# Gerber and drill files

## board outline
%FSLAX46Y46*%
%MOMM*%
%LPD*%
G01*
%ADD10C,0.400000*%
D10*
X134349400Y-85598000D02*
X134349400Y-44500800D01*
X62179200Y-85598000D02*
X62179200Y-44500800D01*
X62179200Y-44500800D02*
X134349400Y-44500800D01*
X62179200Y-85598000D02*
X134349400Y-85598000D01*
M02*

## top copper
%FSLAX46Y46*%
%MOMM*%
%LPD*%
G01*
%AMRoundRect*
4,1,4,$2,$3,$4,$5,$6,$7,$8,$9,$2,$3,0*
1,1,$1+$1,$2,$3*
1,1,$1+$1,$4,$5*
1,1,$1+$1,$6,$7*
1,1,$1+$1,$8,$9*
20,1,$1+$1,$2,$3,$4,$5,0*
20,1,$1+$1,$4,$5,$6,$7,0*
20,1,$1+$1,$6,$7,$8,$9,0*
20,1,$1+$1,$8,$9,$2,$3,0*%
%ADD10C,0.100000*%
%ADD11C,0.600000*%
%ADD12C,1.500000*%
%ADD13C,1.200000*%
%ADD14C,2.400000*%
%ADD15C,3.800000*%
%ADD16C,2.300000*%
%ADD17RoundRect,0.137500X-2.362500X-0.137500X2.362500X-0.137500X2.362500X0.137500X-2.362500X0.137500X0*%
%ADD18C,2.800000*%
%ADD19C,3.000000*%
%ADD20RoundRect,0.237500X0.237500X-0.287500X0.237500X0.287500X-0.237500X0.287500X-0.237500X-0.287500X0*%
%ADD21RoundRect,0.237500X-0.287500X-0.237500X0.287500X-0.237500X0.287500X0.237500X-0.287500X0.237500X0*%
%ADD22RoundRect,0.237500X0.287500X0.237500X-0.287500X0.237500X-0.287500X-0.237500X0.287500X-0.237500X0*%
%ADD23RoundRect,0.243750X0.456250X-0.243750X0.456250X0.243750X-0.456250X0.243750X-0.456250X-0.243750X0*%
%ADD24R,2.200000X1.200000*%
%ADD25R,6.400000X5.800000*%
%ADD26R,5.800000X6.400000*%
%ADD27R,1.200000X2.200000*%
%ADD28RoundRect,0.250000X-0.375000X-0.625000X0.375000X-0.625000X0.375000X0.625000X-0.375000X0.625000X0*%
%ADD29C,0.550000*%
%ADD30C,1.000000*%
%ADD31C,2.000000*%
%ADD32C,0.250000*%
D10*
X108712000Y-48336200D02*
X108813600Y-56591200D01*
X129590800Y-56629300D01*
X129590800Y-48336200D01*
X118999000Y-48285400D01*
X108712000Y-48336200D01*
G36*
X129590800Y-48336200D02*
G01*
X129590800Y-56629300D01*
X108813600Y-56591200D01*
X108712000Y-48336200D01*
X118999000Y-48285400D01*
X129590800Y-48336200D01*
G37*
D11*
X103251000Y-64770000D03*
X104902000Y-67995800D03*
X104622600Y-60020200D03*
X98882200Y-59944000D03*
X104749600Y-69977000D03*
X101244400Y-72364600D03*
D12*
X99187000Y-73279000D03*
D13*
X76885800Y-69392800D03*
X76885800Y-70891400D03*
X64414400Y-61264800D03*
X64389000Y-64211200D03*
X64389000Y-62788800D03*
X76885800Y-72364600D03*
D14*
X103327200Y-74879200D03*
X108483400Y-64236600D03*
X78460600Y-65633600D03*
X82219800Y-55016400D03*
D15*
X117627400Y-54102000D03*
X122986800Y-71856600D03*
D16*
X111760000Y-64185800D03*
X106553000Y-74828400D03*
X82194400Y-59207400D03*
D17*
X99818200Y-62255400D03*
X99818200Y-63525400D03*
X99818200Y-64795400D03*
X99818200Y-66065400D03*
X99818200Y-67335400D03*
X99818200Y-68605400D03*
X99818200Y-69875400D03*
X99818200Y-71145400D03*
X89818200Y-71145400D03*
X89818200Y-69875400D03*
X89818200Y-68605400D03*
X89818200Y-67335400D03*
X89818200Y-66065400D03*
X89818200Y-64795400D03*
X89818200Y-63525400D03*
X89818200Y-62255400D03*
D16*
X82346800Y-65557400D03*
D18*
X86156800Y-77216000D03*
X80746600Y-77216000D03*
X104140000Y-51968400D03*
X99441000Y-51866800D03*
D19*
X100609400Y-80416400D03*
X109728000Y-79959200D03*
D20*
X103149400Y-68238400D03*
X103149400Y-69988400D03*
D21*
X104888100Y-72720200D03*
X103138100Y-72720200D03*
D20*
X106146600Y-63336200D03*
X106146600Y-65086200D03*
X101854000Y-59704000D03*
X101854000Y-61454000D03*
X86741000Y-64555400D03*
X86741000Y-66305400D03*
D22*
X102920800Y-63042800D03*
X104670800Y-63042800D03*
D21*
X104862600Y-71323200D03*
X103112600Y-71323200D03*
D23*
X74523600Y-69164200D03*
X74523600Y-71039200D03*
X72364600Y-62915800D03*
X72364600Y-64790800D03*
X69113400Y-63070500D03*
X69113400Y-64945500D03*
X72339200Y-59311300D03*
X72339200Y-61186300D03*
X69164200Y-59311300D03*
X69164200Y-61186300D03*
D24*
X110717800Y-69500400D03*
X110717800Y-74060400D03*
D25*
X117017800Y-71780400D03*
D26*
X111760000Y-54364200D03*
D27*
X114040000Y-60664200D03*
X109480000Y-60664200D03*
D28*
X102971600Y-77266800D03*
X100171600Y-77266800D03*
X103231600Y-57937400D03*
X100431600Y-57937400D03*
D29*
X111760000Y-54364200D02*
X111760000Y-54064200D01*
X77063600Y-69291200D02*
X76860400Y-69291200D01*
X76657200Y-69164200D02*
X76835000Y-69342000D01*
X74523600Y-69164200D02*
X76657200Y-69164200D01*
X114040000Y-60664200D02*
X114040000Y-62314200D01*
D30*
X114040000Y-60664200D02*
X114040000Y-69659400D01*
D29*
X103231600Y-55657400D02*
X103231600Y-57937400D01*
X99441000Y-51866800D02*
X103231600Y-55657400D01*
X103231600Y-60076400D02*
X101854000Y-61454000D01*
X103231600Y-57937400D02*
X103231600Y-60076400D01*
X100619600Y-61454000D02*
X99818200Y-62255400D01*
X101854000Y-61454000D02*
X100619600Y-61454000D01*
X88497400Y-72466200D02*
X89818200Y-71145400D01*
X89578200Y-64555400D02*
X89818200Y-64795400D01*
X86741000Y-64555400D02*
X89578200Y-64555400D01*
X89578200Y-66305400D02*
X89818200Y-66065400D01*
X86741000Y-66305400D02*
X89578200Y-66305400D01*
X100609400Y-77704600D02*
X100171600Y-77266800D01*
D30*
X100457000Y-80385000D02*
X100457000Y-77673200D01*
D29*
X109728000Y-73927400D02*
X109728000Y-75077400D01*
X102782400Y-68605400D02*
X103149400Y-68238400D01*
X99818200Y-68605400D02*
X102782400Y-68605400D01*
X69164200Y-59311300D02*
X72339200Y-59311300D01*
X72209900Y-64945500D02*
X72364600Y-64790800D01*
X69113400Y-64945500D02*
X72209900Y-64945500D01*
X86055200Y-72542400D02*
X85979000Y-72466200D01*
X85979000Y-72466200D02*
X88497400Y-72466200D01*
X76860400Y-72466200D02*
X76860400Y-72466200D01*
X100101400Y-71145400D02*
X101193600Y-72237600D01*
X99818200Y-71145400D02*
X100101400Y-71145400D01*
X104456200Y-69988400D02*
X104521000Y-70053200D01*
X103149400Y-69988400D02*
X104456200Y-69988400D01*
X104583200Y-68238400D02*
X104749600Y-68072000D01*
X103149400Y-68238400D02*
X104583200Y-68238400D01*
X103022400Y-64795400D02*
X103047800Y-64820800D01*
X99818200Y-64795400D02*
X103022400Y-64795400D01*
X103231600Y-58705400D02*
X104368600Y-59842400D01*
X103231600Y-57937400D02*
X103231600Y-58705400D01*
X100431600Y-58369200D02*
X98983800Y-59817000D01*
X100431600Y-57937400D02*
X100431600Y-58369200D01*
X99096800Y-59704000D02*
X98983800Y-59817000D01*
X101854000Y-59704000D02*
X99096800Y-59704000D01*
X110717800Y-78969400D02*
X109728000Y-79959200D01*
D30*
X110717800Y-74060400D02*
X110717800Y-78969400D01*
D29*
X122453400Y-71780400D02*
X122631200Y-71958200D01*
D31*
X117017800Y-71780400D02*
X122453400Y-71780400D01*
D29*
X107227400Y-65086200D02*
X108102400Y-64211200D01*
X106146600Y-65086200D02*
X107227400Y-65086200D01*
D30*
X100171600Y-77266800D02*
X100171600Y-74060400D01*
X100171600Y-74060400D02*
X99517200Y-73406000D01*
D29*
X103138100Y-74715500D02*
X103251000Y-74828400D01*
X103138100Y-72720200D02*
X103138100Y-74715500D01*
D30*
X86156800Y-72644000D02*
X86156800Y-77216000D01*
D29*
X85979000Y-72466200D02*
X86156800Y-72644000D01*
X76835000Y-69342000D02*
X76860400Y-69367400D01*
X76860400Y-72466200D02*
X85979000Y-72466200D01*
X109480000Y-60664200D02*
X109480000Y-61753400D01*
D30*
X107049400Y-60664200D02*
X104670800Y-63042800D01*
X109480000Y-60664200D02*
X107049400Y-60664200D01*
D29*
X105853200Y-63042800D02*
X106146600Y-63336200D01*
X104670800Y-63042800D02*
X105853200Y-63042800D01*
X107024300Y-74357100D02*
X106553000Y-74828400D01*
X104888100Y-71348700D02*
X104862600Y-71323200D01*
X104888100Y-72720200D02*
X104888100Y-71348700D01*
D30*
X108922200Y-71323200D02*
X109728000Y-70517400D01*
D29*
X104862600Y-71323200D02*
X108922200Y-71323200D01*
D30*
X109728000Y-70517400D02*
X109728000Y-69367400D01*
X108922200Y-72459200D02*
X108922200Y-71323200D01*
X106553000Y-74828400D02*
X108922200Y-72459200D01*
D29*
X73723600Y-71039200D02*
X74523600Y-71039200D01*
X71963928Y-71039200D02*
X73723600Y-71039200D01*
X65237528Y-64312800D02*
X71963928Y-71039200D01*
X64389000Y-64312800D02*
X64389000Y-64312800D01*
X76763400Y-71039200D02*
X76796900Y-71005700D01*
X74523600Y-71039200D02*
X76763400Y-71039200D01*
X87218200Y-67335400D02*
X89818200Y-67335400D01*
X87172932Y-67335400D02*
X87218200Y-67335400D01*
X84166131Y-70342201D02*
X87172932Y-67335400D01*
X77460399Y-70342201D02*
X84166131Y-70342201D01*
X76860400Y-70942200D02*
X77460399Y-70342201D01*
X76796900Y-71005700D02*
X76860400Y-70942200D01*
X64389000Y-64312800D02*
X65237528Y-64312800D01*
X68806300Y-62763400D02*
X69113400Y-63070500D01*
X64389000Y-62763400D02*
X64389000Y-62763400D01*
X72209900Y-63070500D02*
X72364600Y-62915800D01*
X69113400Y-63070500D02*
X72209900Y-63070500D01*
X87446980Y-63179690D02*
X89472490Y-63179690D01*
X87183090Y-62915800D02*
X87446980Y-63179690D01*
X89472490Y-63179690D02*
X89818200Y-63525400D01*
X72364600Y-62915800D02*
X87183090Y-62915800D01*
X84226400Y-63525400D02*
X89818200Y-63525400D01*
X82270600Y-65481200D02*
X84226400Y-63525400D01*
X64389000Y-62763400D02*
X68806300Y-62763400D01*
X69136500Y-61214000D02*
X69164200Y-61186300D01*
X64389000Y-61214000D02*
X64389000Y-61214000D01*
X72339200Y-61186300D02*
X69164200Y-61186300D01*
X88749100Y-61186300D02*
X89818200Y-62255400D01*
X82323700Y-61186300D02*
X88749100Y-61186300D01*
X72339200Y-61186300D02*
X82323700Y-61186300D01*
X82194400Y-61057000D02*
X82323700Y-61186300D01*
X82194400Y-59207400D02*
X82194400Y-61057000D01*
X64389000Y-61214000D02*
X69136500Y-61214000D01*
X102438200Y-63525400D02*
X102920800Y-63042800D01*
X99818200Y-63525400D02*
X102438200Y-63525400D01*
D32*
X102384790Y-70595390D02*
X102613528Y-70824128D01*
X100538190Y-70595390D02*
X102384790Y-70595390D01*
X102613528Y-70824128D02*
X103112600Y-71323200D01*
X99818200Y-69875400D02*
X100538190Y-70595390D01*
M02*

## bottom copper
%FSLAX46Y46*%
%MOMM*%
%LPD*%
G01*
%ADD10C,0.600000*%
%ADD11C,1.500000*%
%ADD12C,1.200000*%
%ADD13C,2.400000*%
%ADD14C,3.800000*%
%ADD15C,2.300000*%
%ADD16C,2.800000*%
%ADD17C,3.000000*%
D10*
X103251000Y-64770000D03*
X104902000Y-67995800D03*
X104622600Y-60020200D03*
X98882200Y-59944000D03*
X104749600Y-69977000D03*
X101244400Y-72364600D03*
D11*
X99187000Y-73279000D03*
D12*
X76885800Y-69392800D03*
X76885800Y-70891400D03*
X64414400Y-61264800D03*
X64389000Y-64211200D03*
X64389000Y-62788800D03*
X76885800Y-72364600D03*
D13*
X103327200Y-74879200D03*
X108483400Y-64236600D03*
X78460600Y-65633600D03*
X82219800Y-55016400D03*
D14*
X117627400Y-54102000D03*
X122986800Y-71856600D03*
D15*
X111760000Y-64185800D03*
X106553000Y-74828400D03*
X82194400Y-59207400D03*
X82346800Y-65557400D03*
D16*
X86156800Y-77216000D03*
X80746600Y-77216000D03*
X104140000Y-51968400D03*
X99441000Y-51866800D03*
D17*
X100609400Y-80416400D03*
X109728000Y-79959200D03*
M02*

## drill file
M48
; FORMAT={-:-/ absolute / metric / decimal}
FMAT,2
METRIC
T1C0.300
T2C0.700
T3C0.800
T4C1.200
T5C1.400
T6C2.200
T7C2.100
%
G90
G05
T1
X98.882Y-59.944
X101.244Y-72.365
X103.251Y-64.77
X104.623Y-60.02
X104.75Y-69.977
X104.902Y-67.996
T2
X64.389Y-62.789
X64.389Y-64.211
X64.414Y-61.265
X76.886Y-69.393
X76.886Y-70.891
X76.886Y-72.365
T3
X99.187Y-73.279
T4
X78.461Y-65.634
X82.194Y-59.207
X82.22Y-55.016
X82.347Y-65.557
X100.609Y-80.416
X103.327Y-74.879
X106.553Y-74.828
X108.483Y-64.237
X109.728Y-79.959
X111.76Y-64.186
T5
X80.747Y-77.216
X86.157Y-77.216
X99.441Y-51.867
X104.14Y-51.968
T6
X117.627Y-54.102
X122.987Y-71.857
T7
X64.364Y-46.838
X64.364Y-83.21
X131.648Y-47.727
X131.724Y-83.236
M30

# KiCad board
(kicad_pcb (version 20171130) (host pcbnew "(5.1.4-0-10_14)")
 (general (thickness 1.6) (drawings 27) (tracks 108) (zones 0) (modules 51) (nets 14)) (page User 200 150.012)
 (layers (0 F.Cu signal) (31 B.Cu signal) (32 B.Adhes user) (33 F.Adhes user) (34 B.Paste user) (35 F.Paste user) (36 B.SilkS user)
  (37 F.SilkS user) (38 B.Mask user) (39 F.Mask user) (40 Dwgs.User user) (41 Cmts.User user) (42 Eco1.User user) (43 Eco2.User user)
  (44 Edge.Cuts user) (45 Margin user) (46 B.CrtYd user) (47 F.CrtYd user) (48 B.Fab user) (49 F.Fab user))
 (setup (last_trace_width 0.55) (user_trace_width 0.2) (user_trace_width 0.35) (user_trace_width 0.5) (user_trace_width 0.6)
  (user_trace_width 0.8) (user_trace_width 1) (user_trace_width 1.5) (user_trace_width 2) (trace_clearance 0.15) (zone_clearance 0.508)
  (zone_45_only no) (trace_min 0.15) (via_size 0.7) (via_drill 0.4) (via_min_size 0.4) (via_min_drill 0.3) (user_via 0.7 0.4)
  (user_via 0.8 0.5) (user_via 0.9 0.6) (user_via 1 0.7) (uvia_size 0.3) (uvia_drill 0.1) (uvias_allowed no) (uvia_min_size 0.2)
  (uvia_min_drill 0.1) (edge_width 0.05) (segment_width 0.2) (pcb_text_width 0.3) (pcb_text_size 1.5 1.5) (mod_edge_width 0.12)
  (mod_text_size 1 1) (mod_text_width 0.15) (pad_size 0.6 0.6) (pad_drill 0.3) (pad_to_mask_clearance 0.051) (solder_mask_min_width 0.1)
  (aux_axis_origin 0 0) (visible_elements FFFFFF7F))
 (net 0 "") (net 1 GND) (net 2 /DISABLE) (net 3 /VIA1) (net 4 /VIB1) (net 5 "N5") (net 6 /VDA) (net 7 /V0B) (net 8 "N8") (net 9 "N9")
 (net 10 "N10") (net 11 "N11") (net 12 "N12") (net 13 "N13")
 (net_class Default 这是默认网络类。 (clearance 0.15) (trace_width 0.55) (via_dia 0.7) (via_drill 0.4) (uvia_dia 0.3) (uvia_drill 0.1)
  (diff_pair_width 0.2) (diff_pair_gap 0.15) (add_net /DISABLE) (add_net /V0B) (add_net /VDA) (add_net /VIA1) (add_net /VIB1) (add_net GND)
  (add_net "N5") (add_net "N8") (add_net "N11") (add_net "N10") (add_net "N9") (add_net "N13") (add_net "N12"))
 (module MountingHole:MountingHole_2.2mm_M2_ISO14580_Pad (layer F.Cu) (at 103.251 64.77)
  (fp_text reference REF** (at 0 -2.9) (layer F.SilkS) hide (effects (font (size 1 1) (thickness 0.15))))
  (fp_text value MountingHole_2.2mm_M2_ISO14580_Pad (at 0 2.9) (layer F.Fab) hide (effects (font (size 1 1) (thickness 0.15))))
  (pad 1 thru_hole circle (at 0 0) (size 0.6 0.6) (drill 0.3) (layers *.Cu *.Mask) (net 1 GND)))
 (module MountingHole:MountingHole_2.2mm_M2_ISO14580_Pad (layer F.Cu) (at 104.902 67.9958)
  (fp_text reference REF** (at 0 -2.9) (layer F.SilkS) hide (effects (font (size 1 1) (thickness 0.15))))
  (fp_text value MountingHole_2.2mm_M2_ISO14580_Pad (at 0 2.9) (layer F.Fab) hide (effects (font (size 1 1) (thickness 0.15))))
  (pad 1 thru_hole circle (at 0 0) (size 0.6 0.6) (drill 0.3) (layers *.Cu *.Mask) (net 1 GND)))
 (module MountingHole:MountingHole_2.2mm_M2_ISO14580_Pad (layer F.Cu) (at 104.6226 60.0202)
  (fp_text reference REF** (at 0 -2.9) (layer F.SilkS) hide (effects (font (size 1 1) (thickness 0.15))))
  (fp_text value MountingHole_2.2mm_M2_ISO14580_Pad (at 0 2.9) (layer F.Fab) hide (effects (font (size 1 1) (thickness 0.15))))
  (pad 1 thru_hole circle (at 0 0) (size 0.6 0.6) (drill 0.3) (layers *.Cu *.Mask) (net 1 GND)))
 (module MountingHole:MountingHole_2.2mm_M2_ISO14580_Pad (layer F.Cu) (at 98.8822 59.944)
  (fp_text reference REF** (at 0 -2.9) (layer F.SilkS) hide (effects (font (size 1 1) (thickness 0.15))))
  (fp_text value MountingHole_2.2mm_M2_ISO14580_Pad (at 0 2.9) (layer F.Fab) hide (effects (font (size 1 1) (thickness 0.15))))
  (pad 1 thru_hole circle (at 0 0) (size 0.6 0.6) (drill 0.3) (layers *.Cu *.Mask) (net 1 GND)))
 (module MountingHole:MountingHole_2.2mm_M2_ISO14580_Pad (layer F.Cu) (at 104.7496 69.977)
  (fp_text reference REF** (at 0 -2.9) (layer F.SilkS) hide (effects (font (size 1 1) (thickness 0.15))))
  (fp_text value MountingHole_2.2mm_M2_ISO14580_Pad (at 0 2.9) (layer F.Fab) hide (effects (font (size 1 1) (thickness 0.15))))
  (pad 1 thru_hole circle (at 0 0) (size 0.6 0.6) (drill 0.3) (layers *.Cu *.Mask) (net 1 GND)))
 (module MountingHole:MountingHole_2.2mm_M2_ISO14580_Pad (layer F.Cu) (at 101.2444 72.3646)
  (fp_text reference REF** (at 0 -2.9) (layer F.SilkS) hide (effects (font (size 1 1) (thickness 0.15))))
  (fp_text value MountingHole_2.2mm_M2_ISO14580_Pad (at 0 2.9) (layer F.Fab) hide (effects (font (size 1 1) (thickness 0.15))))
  (pad 1 thru_hole circle (at 0 0) (size 0.6 0.6) (drill 0.3) (layers *.Cu *.Mask) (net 1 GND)))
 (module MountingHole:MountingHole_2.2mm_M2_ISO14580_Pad (layer F.Cu) (at 99.187 73.279)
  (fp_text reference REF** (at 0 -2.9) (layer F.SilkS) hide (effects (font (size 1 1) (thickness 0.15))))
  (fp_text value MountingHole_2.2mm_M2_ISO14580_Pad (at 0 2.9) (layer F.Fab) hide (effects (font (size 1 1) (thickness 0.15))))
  (pad 1 thru_hole circle (at 0 0) (size 1.5 1.5) (drill 0.8) (layers *.Cu *.Mask) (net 1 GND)))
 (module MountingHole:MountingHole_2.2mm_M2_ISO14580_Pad (layer F.Cu) (at 76.8858 69.3928)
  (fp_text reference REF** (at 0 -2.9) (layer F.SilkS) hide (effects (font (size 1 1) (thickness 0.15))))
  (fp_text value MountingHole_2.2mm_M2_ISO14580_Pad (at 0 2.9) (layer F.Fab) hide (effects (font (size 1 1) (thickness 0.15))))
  (pad 1 thru_hole circle (at 0 0) (size 1.2 1.2) (drill 0.7) (layers *.Cu *.Mask) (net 1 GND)))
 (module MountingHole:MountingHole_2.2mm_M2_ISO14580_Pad (layer F.Cu) (at 76.8858 70.8914)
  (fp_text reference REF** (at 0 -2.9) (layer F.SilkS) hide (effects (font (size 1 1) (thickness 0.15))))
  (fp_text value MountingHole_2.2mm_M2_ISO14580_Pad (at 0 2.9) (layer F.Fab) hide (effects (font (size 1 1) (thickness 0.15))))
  (pad 1 thru_hole circle (at 0 0) (size 1.2 1.2) (drill 0.7) (layers *.Cu *.Mask) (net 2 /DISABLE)))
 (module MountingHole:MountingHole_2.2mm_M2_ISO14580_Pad (layer F.Cu) (at 64.4144 61.2648)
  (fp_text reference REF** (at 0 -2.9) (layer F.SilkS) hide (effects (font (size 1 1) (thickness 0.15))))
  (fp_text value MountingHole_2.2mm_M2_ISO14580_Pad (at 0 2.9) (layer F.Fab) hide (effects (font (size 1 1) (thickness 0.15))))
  (pad 1 thru_hole circle (at 0 0) (size 1.2 1.2) (drill 0.7) (layers *.Cu *.Mask) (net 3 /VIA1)))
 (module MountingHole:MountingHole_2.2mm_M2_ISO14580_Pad (layer F.Cu) (at 64.389 64.2112)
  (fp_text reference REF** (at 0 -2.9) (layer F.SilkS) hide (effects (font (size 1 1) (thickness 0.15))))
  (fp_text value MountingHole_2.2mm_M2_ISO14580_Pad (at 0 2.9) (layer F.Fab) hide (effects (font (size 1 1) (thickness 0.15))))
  (pad 1 thru_hole circle (at 0 0) (size 1.2 1.2) (drill 0.7) (layers *.Cu *.Mask) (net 2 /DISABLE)))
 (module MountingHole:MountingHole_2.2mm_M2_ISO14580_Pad (layer F.Cu) (at 64.389 62.7888)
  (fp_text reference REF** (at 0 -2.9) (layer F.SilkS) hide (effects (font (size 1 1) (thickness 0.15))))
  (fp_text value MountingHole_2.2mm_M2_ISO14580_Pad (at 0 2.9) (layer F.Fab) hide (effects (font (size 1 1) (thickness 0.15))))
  (pad 1 thru_hole circle (at 0 0) (size 1.2 1.2) (drill 0.7) (layers *.Cu *.Mask) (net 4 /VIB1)))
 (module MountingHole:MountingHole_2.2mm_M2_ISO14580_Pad (layer F.Cu) (at 76.8858 72.3646)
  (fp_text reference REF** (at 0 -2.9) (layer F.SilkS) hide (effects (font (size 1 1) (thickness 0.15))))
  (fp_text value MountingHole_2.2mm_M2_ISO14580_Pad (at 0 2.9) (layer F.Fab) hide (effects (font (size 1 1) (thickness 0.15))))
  (pad 1 thru_hole circle (at 0 0) (size 1.2 1.2) (drill 0.7) (layers *.Cu *.Mask) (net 1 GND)))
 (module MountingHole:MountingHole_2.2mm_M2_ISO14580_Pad (layer F.Cu) (at 103.3272 74.8792)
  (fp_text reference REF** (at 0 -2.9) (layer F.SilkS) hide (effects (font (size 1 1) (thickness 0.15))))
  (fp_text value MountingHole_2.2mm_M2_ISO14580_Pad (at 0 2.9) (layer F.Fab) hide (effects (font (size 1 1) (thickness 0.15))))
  (pad 1 thru_hole circle (at 0 0) (size 2.4 2.4) (drill 1.2) (layers *.Cu *.Mask) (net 1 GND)))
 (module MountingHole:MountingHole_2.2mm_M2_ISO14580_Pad (layer F.Cu) (at 108.4834 64.2366)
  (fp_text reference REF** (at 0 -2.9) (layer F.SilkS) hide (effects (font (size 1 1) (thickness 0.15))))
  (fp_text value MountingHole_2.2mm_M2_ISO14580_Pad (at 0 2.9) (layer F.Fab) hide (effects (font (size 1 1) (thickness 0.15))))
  (pad 1 thru_hole circle (at 0 0) (size 2.4 2.4) (drill 1.2) (layers *.Cu *.Mask) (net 1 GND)))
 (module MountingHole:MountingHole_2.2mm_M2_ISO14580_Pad (layer F.Cu) (at 78.4606 65.6336)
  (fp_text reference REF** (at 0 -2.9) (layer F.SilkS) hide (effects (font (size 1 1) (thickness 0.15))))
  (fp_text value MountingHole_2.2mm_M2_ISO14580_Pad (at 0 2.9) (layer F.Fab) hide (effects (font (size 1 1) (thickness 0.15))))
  (pad 1 thru_hole circle (at 0 0) (size 2.4 2.4) (drill 1.2) (layers *.Cu *.Mask) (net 1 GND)))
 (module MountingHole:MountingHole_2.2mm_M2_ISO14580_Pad (layer F.Cu) (at 82.2198 55.0164)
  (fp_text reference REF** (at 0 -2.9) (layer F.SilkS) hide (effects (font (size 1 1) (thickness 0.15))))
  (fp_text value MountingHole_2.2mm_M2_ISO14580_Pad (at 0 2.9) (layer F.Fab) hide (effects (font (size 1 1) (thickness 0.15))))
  (pad 1 thru_hole circle (at 0 0) (size 2.4 2.4) (drill 1.2) (layers *.Cu *.Mask) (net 1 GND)))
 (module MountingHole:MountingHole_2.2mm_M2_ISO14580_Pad (layer F.Cu) (at 117.6274 54.102)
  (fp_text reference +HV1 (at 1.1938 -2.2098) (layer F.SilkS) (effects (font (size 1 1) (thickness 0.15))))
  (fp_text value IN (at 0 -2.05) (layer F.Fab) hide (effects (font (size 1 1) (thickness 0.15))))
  (pad 1 thru_hole circle (at 0 0) (size 3.8 3.8) (drill 2.2) (layers *.Cu *.Mask) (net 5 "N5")))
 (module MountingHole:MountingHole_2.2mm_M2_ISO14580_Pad (layer F.Cu) (at 122.9868 71.8566)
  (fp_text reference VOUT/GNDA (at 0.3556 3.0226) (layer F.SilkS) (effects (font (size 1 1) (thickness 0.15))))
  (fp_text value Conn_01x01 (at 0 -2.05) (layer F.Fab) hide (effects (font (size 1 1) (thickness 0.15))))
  (pad 1 thru_hole circle (at 0 0) (size 3.8 3.8) (drill 2.2) (layers *.Cu *.Mask) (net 1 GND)))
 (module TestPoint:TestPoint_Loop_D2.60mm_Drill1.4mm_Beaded (layer F.Cu) (at 111.76 64.1858)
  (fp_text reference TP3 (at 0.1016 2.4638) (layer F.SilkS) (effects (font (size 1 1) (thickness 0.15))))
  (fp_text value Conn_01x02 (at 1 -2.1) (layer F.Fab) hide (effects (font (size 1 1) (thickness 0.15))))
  (pad 1 thru_hole circle (at 0 0) (size 2.3 2.3) (drill 1.2) (layers *.Cu *.Mask) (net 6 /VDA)))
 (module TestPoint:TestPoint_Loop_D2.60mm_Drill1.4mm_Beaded (layer F.Cu) (at 106.553 74.8284)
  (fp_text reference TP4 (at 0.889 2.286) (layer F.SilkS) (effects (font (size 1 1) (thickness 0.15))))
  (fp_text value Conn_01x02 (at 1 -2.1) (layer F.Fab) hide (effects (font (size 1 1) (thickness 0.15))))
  (pad 1 thru_hole circle (at 0 0) (size 2.3 2.3) (drill 1.2) (layers *.Cu *.Mask) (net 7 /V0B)))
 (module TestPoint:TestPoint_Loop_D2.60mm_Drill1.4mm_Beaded (layer F.Cu) (at 82.1944 59.2074 90)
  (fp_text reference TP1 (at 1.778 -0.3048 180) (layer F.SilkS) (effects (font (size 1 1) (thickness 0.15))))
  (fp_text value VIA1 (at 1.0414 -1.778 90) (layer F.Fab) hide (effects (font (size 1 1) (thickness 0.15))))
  (pad 1 thru_hole circle (at 0 0 90) (size 2.3 2.3) (drill 1.2) (layers *.Cu *.Mask) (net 3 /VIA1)))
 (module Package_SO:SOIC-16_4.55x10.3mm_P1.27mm (layer F.Cu) (at 94.8182 66.7004)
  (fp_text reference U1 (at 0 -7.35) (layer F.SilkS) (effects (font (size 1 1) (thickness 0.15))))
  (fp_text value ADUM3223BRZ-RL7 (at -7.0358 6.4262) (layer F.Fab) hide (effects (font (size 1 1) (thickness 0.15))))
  (pad 16 smd roundrect (at 5 -4.445) (size 5 0.55) (layers F.Cu F.Paste F.Mask) (roundrect_rratio 0.25) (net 1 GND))
  (pad 15 smd roundrect (at 5 -3.175) (size 5 0.55) (layers F.Cu F.Paste F.Mask) (roundrect_rratio 0.25) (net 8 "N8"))
  (pad 14 smd roundrect (at 5 -1.905) (size 5 0.55) (layers F.Cu F.Paste F.Mask) (roundrect_rratio 0.25) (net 1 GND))
  (pad 13 smd roundrect (at 5 -0.635) (size 5 0.55) (layers F.Cu F.Paste F.Mask) (roundrect_rratio 0.25) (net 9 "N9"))
  (pad 12 smd roundrect (at 5 0.635) (size 5 0.55) (layers F.Cu F.Paste F.Mask) (roundrect_rratio 0.25) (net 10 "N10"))
  (pad 11 smd roundrect (at 5 1.905) (size 5 0.55) (layers F.Cu F.Paste F.Mask) (roundrect_rratio 0.25) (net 1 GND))
  (pad 10 smd roundrect (at 5 3.175) (size 5 0.55) (layers F.Cu F.Paste F.Mask) (roundrect_rratio 0.25) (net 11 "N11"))
  (pad 9 smd roundrect (at 5 4.445) (size 5 0.55) (layers F.Cu F.Paste F.Mask) (roundrect_rratio 0.25) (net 1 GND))
  (pad 8 smd roundrect (at -5 4.445) (size 5 0.55) (layers F.Cu F.Paste F.Mask) (roundrect_rratio 0.25) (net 1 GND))
  (pad 7 smd roundrect (at -5 3.175) (size 5 0.55) (layers F.Cu F.Paste F.Mask) (roundrect_rratio 0.25) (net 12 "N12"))
  (pad 6 smd roundrect (at -5 1.905) (size 5 0.55) (layers F.Cu F.Paste F.Mask) (roundrect_rratio 0.25) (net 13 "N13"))
  (pad 5 smd roundrect (at -5 0.635) (size 5 0.55) (layers F.Cu F.Paste F.Mask) (roundrect_rratio 0.25) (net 2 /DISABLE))
  (pad 4 smd roundrect (at -5 -0.635) (size 5 0.55) (layers F.Cu F.Paste F.Mask) (roundrect_rratio 0.25) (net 1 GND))
  (pad 3 smd roundrect (at -5 -1.905) (size 5 0.55) (layers F.Cu F.Paste F.Mask) (roundrect_rratio 0.25) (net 1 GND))
  (pad 2 smd roundrect (at -5 -3.175) (size 5 0.55) (layers F.Cu F.Paste F.Mask) (roundrect_rratio 0.25) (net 4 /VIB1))
  (pad 1 smd roundrect (at -5 -4.445) (size 5 0.55) (layers F.Cu F.Paste F.Mask) (roundrect_rratio 0.25) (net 3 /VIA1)))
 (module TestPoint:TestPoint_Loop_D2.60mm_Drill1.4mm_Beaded (layer F.Cu) (at 82.3468 65.5574 180)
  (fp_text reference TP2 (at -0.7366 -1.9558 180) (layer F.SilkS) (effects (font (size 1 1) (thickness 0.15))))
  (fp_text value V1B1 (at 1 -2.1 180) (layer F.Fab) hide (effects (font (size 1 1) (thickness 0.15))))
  (pad 1 thru_hole circle (at 0 0 180) (size 2.3 2.3) (drill 1.2) (layers *.Cu *.Mask) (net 4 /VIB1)))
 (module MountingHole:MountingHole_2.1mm (layer F.Cu) (at 131.6482 47.7266)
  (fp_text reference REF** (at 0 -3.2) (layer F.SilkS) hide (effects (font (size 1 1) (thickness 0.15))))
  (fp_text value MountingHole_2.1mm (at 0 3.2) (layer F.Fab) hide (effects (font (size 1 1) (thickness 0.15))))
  (pad "" np_thru_hole circle (at 0 0) (size 2.1 2.1) (drill 2.1) (layers *.Cu *.Mask)))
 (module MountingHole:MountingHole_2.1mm (layer F.Cu) (at 131.7752 83.2358)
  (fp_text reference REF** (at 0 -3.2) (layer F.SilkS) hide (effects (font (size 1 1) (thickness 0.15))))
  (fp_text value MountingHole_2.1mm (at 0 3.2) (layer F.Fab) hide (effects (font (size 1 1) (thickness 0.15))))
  (pad "" np_thru_hole circle (at -0.0508 0) (size 2.1 2.1) (drill 2.1) (layers *.Cu *.Mask)))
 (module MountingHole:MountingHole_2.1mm (layer F.Cu) (at 64.3636 83.2104)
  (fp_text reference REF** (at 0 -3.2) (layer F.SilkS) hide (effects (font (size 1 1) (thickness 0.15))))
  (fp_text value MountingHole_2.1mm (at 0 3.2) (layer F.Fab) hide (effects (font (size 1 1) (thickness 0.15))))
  (pad "" np_thru_hole circle (at 0 0) (size 2.1 2.1) (drill 2.1) (layers *.Cu *.Mask)))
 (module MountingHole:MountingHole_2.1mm (layer F.Cu) (at 64.3636 46.8376)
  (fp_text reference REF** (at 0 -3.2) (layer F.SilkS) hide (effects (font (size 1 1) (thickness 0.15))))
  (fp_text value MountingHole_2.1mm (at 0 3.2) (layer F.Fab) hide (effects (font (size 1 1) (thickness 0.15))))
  (pad "" np_thru_hole circle (at 0 0) (size 2.1 2.1) (drill 2.1) (layers *.Cu *.Mask)))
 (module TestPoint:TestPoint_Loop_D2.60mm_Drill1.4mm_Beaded (layer F.Cu) (at 86.1568 77.216)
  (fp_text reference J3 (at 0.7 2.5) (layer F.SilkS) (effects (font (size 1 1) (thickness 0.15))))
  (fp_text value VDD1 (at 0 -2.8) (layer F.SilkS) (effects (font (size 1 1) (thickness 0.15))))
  (pad 1 thru_hole circle (at 0 0) (size 2.8 2.8) (drill 1.4) (layers *.Cu *.Mask) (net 1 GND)))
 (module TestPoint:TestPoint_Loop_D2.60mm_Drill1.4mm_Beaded (layer F.Cu) (at 80.7466 77.216)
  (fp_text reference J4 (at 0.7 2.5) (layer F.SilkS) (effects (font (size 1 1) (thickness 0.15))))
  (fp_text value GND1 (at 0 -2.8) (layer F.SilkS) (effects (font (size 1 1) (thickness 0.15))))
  (pad 1 thru_hole circle (at 0 0) (size 2.8 2.8) (drill 1.4) (layers *.Cu *.Mask) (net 1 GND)))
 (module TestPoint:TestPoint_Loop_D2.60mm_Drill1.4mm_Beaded (layer F.Cu) (at 104.14 51.9684)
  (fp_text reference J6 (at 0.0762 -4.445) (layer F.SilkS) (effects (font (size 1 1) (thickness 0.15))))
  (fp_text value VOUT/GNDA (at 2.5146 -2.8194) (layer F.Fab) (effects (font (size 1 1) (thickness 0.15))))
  (pad 1 thru_hole circle (at 0 0) (size 2.8 2.8) (drill 1.4) (layers *.Cu *.Mask)))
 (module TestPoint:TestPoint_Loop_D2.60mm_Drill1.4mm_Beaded (layer F.Cu) (at 99.441 51.8668)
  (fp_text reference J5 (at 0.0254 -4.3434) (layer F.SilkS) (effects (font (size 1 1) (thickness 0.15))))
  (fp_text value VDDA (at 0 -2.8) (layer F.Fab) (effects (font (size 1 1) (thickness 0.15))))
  (pad 1 thru_hole circle (at 0 0) (size 2.8 2.8) (drill 1.4) (layers *.Cu *.Mask) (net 1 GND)))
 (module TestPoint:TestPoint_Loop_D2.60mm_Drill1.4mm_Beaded (layer F.Cu) (at 100.6094 80.4164)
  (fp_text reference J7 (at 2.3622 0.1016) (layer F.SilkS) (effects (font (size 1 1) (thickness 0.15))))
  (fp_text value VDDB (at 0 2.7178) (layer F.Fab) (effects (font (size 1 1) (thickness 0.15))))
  (pad 1 thru_hole circle (at 0 0) (size 3 3) (drill 1.2) (layers *.Cu *.Mask) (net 1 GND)))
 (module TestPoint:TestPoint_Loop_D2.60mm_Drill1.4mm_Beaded (layer F.Cu) (at 109.728 79.9592)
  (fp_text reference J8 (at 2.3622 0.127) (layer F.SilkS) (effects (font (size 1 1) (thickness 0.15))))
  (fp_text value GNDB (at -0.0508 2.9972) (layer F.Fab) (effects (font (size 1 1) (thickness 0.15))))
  (pad 1 thru_hole circle (at 0 0) (size 3 3) (drill 1.2) (layers *.Cu *.Mask) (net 1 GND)))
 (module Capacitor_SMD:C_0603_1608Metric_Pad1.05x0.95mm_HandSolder (layer F.Cu) (at 103.1494 69.1134 90)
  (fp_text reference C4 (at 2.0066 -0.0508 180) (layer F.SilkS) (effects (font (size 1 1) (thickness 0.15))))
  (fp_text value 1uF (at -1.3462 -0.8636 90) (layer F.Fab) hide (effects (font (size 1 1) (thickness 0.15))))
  (pad 2 smd roundrect (at 0.875 0 90) (size 1.05 0.95) (layers F.Cu F.Paste F.Mask) (roundrect_rratio 0.25) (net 1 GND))
  (pad 1 smd roundrect (at -0.875 0 90) (size 1.05 0.95) (layers F.Cu F.Paste F.Mask) (roundrect_rratio 0.25) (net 1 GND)))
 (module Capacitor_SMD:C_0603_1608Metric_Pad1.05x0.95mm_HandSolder (layer F.Cu) (at 104.0131 72.7202)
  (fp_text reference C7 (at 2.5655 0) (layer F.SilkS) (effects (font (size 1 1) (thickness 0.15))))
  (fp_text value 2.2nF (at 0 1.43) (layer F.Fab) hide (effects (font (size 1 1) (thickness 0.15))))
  (pad 2 smd roundrect (at 0.875 0) (size 1.05 0.95) (layers F.Cu F.Paste F.Mask) (roundrect_rratio 0.25) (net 7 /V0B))
  (pad 1 smd roundrect (at -0.875 0) (size 1.05 0.95) (layers F.Cu F.Paste F.Mask) (roundrect_rratio 0.25) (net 1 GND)))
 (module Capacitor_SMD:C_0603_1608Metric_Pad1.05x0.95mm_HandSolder (layer F.Cu) (at 106.1466 64.2112 90)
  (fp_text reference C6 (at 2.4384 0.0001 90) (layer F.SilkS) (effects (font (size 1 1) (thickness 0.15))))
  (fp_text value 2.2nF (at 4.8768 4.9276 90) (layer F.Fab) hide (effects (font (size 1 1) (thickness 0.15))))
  (pad 2 smd roundrect (at 0.875 0 90) (size 1.05 0.95) (layers F.Cu F.Paste F.Mask) (roundrect_rratio 0.25) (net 6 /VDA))
  (pad 1 smd roundrect (at -0.875 0 90) (size 1.05 0.95) (layers F.Cu F.Paste F.Mask) (roundrect_rratio 0.25) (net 1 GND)))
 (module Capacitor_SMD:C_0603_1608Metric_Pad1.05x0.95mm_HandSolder (layer F.Cu) (at 101.854 60.579 90)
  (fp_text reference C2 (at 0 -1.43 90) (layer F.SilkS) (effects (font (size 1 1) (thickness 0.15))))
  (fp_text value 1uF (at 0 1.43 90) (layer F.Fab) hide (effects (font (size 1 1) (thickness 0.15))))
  (pad 2 smd roundrect (at 0.875 0 90) (size 1.05 0.95) (layers F.Cu F.Paste F.Mask) (roundrect_rratio 0.25) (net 1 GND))
  (pad 1 smd roundrect (at -0.875 0 90) (size 1.05 0.95) (layers F.Cu F.Paste F.Mask) (roundrect_rratio 0.25) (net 1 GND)))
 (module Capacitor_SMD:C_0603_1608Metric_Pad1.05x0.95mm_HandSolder (layer F.Cu) (at 86.741 65.4304 90)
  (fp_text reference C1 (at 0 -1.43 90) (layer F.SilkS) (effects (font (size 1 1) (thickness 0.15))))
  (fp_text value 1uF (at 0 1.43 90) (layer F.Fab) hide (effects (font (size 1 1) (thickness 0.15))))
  (pad 2 smd roundrect (at 0.875 0 90) (size 1.05 0.95) (layers F.Cu F.Paste F.Mask) (roundrect_rratio 0.25) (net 1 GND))
  (pad 1 smd roundrect (at -0.875 0 90) (size 1.05 0.95) (layers F.Cu F.Paste F.Mask) (roundrect_rratio 0.25) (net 1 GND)))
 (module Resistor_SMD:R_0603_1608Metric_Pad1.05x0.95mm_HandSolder (layer F.Cu) (at 103.7958 63.0428 180)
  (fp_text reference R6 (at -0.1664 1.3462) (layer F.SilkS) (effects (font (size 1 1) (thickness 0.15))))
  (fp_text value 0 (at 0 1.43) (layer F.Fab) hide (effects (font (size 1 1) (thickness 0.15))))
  (pad 2 smd roundrect (at 0.875 0 180) (size 1.05 0.95) (layers F.Cu F.Paste F.Mask) (roundrect_rratio 0.25) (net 8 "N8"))
  (pad 1 smd roundrect (at -0.875 0 180) (size 1.05 0.95) (layers F.Cu F.Paste F.Mask) (roundrect_rratio 0.25) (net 6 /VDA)))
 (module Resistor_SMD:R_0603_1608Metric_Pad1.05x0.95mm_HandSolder (layer F.Cu) (at 103.9876 71.3232)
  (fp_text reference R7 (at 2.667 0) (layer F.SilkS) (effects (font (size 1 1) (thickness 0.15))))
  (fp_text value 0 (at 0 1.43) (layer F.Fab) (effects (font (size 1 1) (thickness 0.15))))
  (pad 2 smd roundrect (at 0.875 0) (size 1.05 0.95) (layers F.Cu F.Paste F.Mask) (roundrect_rratio 0.25) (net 7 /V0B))
  (pad 1 smd roundrect (at -0.875 0) (size 1.05 0.95) (layers F.Cu F.Paste F.Mask) (roundrect_rratio 0.25) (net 11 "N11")))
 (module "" (layer F.Cu) (at 64.7446 49.2506 90)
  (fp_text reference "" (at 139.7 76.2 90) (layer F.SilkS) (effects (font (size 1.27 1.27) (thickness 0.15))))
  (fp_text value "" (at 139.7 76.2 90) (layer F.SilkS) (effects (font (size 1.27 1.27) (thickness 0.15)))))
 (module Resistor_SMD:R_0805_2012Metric (layer F.Cu) (at 74.5236 70.1017 90)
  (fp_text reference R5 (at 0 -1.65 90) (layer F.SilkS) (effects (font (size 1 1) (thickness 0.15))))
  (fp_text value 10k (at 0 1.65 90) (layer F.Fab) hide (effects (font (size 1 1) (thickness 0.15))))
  (pad 2 smd roundrect (at 0.9375 0 90) (size 0.975 1.4) (layers F.Cu F.Paste F.Mask) (roundrect_rratio 0.25) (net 1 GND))
  (pad 1 smd roundrect (at -0.9375 0 90) (size 0.975 1.4) (layers F.Cu F.Paste F.Mask) (roundrect_rratio 0.25) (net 2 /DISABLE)))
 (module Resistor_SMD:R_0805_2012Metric (layer F.Cu) (at 72.3646 63.8533 90)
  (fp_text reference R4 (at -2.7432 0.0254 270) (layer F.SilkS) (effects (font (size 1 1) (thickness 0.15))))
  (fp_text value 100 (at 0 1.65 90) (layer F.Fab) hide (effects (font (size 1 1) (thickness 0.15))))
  (pad 2 smd roundrect (at 0.9375 0 90) (size 0.975 1.4) (layers F.Cu F.Paste F.Mask) (roundrect_rratio 0.25) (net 4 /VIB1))
  (pad 1 smd roundrect (at -0.9375 0 90) (size 0.975 1.4) (layers F.Cu F.Paste F.Mask) (roundrect_rratio 0.25) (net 1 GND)))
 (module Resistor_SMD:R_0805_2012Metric (layer F.Cu) (at 69.1134 64.008 90)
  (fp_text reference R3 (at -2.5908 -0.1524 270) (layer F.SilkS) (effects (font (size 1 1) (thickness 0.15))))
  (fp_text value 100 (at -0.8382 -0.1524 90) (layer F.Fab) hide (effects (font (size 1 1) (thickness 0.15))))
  (pad 2 smd roundrect (at 0.9375 0 90) (size 0.975 1.4) (layers F.Cu F.Paste F.Mask) (roundrect_rratio 0.25) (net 4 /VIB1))
  (pad 1 smd roundrect (at -0.9375 0 90) (size 0.975 1.4) (layers F.Cu F.Paste F.Mask) (roundrect_rratio 0.25) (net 1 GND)))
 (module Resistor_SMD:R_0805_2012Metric (layer F.Cu) (at 72.3392 60.2488 90)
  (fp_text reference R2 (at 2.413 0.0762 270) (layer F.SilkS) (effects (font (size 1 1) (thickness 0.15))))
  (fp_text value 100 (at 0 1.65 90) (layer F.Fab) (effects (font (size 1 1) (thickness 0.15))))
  (pad 2 smd roundrect (at 0.9375 0 90) (size 0.975 1.4) (layers F.Cu F.Paste F.Mask) (roundrect_rratio 0.25) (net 1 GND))
  (pad 1 smd roundrect (at -0.9375 0 90) (size 0.975 1.4) (layers F.Cu F.Paste F.Mask) (roundrect_rratio 0.25) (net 3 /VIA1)))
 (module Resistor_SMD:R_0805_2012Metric (layer F.Cu) (at 69.1642 60.2488 90)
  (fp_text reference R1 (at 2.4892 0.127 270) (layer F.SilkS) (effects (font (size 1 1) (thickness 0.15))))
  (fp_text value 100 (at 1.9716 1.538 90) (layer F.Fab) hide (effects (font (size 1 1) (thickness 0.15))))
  (pad 2 smd roundrect (at 0.9375 0 90) (size 0.975 1.4) (layers F.Cu F.Paste F.Mask) (roundrect_rratio 0.25) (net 1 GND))
  (pad 1 smd roundrect (at -0.9375 0 90) (size 0.975 1.4) (layers F.Cu F.Paste F.Mask) (roundrect_rratio 0.25) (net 3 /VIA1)))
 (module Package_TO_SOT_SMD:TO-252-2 (layer F.Cu) (at 114.9178 71.7804)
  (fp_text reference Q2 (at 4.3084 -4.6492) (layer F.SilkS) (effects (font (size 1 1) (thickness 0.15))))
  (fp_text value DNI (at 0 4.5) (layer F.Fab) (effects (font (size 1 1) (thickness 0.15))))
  (pad 1 smd rect (at -4.2 -2.28) (size 2.2 1.2) (layers F.Cu F.Paste F.Mask) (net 7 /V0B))
  (pad 3 smd rect (at -4.2 2.28) (size 2.2 1.2) (layers F.Cu F.Paste F.Mask) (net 1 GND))
  (pad "" smd rect (at 2.1 0) (size 6.4 5.8) (layers F.Cu F.Paste F.Mask))
  (pad "" smd rect (at 3.775 1.525) (size 3.05 2.75) (layers F.Paste))
  (pad "" smd rect (at 0.425 -1.525) (size 3.05 2.75) (layers F.Paste))
  (pad "" smd rect (at 3.775 -1.525) (size 3.05 2.75) (layers F.Paste))
  (pad "" smd rect (at 0.425 1.525) (size 3.05 2.75) (layers F.Paste)))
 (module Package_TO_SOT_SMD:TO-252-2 (layer F.Cu) (at 111.76 56.4642 90)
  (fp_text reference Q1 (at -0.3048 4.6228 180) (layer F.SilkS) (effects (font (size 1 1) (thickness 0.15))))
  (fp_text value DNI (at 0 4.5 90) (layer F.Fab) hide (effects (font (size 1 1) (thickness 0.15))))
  (pad "" smd rect (at 0.425 1.525 90) (size 3.05 2.75) (layers F.Paste))
  (pad "" smd rect (at 3.775 -1.525 90) (size 3.05 2.75) (layers F.Paste))
  (pad "" smd rect (at 0.425 -1.525 90) (size 3.05 2.75) (layers F.Paste))
  (pad "" smd rect (at 3.775 1.525 90) (size 3.05 2.75) (layers F.Paste))
  (pad 2 smd rect (at 2.1 0 90) (size 6.4 5.8) (layers F.Cu F.Mask))
  (pad 3 smd rect (at -4.2 2.28 90) (size 2.2 1.2) (layers F.Cu F.Paste F.Mask) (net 1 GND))
  (pad 1 smd rect (at -4.2 -2.28 90) (size 2.2 1.2) (layers F.Cu F.Paste F.Mask) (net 6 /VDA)))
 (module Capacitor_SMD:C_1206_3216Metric (layer F.Cu) (at 101.5716 77.2668)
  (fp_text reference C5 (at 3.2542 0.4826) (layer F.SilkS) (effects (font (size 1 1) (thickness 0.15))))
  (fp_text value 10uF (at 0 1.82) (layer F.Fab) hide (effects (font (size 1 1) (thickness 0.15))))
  (pad 2 smd roundrect (at 1.4 0) (size 1.25 1.75) (layers F.Cu F.Paste F.Mask) (roundrect_rratio 0.2))
  (pad 1 smd roundrect (at -1.4 0) (size 1.25 1.75) (layers F.Cu F.Paste F.Mask) (roundrect_rratio 0.2) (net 1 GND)))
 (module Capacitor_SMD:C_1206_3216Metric (layer F.Cu) (at 101.8316 57.9374)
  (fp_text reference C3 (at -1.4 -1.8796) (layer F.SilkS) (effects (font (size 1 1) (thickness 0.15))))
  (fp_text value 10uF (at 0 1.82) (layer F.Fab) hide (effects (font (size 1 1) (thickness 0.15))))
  (pad 2 smd roundrect (at 1.4 0) (size 1.25 1.75) (layers F.Cu F.Paste F.Mask) (roundrect_rratio 0.2) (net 1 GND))
  (pad 1 smd roundrect (at -1.4 0) (size 1.25 1.75) (layers F.Cu F.Paste F.Mask) (roundrect_rratio 0.2) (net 1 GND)))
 (gr_line (start 134.3494 85.598) (end 134.3494 44.5008) (layer Edge.Cuts) (width 0.4))
 (gr_line (start 62.1792 85.598) (end 62.1792 44.5008) (layer Edge.Cuts) (width 0.4))
 (gr_line (start 62.1792 44.5008) (end 134.3494 44.5008) (layer Edge.Cuts) (width 0.4))
 (gr_poly
  (pts (xy 108.712 48.3362) (xy 108.8136 56.5912) (xy 129.5908 56.6293) (xy 129.5908 48.3362) (xy 118.999 48.2854)) (layer F.Cu) (width 0.1))
 (gr_line (start 62.1792 85.598) (end 134.3494 85.598) (layer Edge.Cuts) (width 0.4))
 (segment (start 111.76 54.3642) (end 111.76 54.0642) (width 0.55) (layer F.Cu) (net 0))
 (segment (start 77.0636 69.2912) (end 76.8604 69.2912) (width 0.55) (layer F.Cu) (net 1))
 (segment (start 76.6572 69.1642) (end 76.835 69.342) (width 0.55) (layer F.Cu) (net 1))
 (segment (start 74.5236 69.1642) (end 76.6572 69.1642) (width 0.55) (layer F.Cu) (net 1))
 (segment (start 114.04 60.6642) (end 114.04 62.3142) (width 0.55) (layer F.Cu) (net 1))
 (segment (start 114.04 60.6642) (end 114.04 69.6594) (width 1) (layer F.Cu) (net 1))
 (segment (start 103.2316 55.6574) (end 103.2316 57.9374) (width 0.55) (layer F.Cu) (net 1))
 (segment (start 99.441 51.8668) (end 103.2316 55.6574) (width 0.55) (layer F.Cu) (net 1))
 (segment (start 103.2316 60.0764) (end 101.854 61.454) (width 0.55) (layer F.Cu) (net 1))
 (segment (start 103.2316 57.9374) (end 103.2316 60.0764) (width 0.55) (layer F.Cu) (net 1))
 (segment (start 100.6196 61.454) (end 99.8182 62.2554) (width 0.55) (layer F.Cu) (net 1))
 (segment (start 101.854 61.454) (end 100.6196 61.454) (width 0.55) (layer F.Cu) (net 1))
 (segment (start 88.4974 72.4662) (end 89.8182 71.1454) (width 0.55) (layer F.Cu) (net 1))
 (segment (start 89.5782 64.5554) (end 89.8182 64.7954) (width 0.55) (layer F.Cu) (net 1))
 (segment (start 86.741 64.5554) (end 89.5782 64.5554) (width 0.55) (layer F.Cu) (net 1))
 (segment (start 89.5782 66.3054) (end 89.8182 66.0654) (width 0.55) (layer F.Cu) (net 1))
 (segment (start 86.741 66.3054) (end 89.5782 66.3054) (width 0.55) (layer F.Cu) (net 1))
 (segment (start 100.6094 77.7046) (end 100.1716 77.2668) (width 0.55) (layer F.Cu) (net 1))
 (segment (start 100.457 80.385) (end 100.457 77.6732) (width 1) (layer F.Cu) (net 1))
 (segment (start 109.728 73.9274) (end 109.728 75.0774) (width 0.55) (layer F.Cu) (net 1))
 (segment (start 102.7824 68.6054) (end 103.1494 68.2384) (width 0.55) (layer F.Cu) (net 1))
 (segment (start 99.8182 68.6054) (end 102.7824 68.6054) (width 0.55) (layer F.Cu) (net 1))
 (segment (start 69.1642 59.3113) (end 72.3392 59.3113) (width 0.55) (layer F.Cu) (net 1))
 (segment (start 72.2099 64.9455) (end 72.3646 64.7908) (width 0.55) (layer F.Cu) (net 1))
 (segment (start 69.1134 64.9455) (end 72.2099 64.9455) (width 0.55) (layer F.Cu) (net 1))
 (segment (start 86.0552 72.5424) (end 85.979 72.4662) (width 0.55) (layer F.Cu) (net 1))
 (segment (start 85.979 72.4662) (end 88.4974 72.4662) (width 0.55) (layer F.Cu) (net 1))
 (segment (start 76.8604 72.4662) (end 76.8604 72.4662) (width 0.55) (layer F.Cu) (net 1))
 (segment (start 100.1014 71.1454) (end 101.1936 72.2376) (width 0.55) (layer F.Cu) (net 1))
 (segment (start 99.8182 71.1454) (end 100.1014 71.1454) (width 0.55) (layer F.Cu) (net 1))
 (segment (start 104.4562 69.9884) (end 104.521 70.0532) (width 0.55) (layer F.Cu) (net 1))
 (segment (start 103.1494 69.9884) (end 104.4562 69.9884) (width 0.55) (layer F.Cu) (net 1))
 (segment (start 104.5832 68.2384) (end 104.7496 68.072) (width 0.55) (layer F.Cu) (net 1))
 (segment (start 103.1494 68.2384) (end 104.5832 68.2384) (width 0.55) (layer F.Cu) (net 1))
 (segment (start 103.0224 64.7954) (end 103.0478 64.8208) (width 0.55) (layer F.Cu) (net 1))
 (segment (start 99.8182 64.7954) (end 103.0224 64.7954) (width 0.55) (layer F.Cu) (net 1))
 (segment (start 103.2316 58.7054) (end 104.3686 59.8424) (width 0.55) (layer F.Cu) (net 1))
 (segment (start 103.2316 57.9374) (end 103.2316 58.7054) (width 0.55) (layer F.Cu) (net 1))
 (segment (start 100.4316 58.3692) (end 98.9838 59.817) (width 0.55) (layer F.Cu) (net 1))
 (segment (start 100.4316 57.9374) (end 100.4316 58.3692) (width 0.55) (layer F.Cu) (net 1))
 (segment (start 99.0968 59.704) (end 98.9838 59.817) (width 0.55) (layer F.Cu) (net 1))
 (segment (start 101.854 59.704) (end 99.0968 59.704) (width 0.55) (layer F.Cu) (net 1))
 (segment (start 110.7178 78.9694) (end 109.728 79.9592) (width 0.55) (layer F.Cu) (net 1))
 (segment (start 110.7178 74.0604) (end 110.7178 78.9694) (width 1) (layer F.Cu) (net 1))
 (segment (start 122.4534 71.7804) (end 122.6312 71.9582) (width 0.55) (layer F.Cu) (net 1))
 (segment (start 117.0178 71.7804) (end 122.4534 71.7804) (width 2) (layer F.Cu) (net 1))
 (segment (start 107.2274 65.0862) (end 108.1024 64.2112) (width 0.55) (layer F.Cu) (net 1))
 (segment (start 106.1466 65.0862) (end 107.2274 65.0862) (width 0.55) (layer F.Cu) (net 1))
 (segment (start 100.1716 77.2668) (end 100.1716 74.0604) (width 1) (layer F.Cu) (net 1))
 (segment (start 100.1716 74.0604) (end 99.5172 73.406) (width 1) (layer F.Cu) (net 1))
 (segment (start 103.1381 74.7155) (end 103.251 74.8284) (width 0.55) (layer F.Cu) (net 1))
 (segment (start 103.1381 72.7202) (end 103.1381 74.7155) (width 0.55) (layer F.Cu) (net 1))
 (segment (start 86.1568 72.644) (end 86.1568 77.216) (width 1) (layer F.Cu) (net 1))
 (segment (start 85.979 72.4662) (end 86.1568 72.644) (width 0.55) (layer F.Cu) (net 1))
 (segment (start 76.835 69.342) (end 76.8604 69.3674) (width 0.55) (layer F.Cu) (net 1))
 (segment (start 76.8604 72.4662) (end 85.979 72.4662) (width 0.55) (layer F.Cu) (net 1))
 (segment (start 109.48 60.6642) (end 109.48 61.7534) (width 0.55) (layer F.Cu) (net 6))
 (segment (start 107.0494 60.6642) (end 104.6708 63.0428) (width 1) (layer F.Cu) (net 6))
 (segment (start 109.48 60.6642) (end 107.0494 60.6642) (width 1) (layer F.Cu) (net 6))
 (segment (start 105.8532 63.0428) (end 106.1466 63.3362) (width 0.55) (layer F.Cu) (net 6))
 (segment (start 104.6708 63.0428) (end 105.8532 63.0428) (width 0.55) (layer F.Cu) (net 6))
 (segment (start 107.0243 74.3571) (end 106.553 74.8284) (width 0.55) (layer F.Cu) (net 7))
 (segment (start 104.8881 71.3487) (end 104.8626 71.3232) (width 0.55) (layer F.Cu) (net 7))
 (segment (start 104.8881 72.7202) (end 104.8881 71.3487) (width 0.55) (layer F.Cu) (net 7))
 (segment (start 108.9222 71.3232) (end 109.728 70.5174) (width 1) (layer F.Cu) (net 7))
 (segment (start 104.8626 71.3232) (end 108.9222 71.3232) (width 0.55) (layer F.Cu) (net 7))
 (segment (start 109.728 70.5174) (end 109.728 69.3674) (width 1) (layer F.Cu) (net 7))
 (segment (start 108.9222 72.4592) (end 108.9222 71.3232) (width 1) (layer F.Cu) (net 7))
 (segment (start 106.553 74.8284) (end 108.9222 72.4592) (width 1) (layer F.Cu) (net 7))
 (segment (start 73.7236 71.0392) (end 74.5236 71.0392) (width 0.55) (layer F.Cu) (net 2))
 (segment (start 71.963928 71.0392) (end 73.7236 71.0392) (width 0.55) (layer F.Cu) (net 2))
 (segment (start 65.237528 64.3128) (end 71.963928 71.0392) (width 0.55) (layer F.Cu) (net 2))
 (segment (start 64.389 64.3128) (end 64.389 64.3128) (width 0.55) (layer F.Cu) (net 2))
 (segment (start 76.7634 71.0392) (end 76.7969 71.0057) (width 0.55) (layer F.Cu) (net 2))
 (segment (start 74.5236 71.0392) (end 76.7634 71.0392) (width 0.55) (layer F.Cu) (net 2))
 (segment (start 87.2182 67.3354) (end 89.8182 67.3354) (width 0.55) (layer F.Cu) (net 2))
 (segment (start 87.172932 67.3354) (end 87.2182 67.3354) (width 0.55) (layer F.Cu) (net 2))
 (segment (start 84.166131 70.342201) (end 87.172932 67.3354) (width 0.55) (layer F.Cu) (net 2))
 (segment (start 77.460399 70.342201) (end 84.166131 70.342201) (width 0.55) (layer F.Cu) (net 2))
 (segment (start 76.8604 70.9422) (end 77.460399 70.342201) (width 0.55) (layer F.Cu) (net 2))
 (segment (start 76.7969 71.0057) (end 76.8604 70.9422) (width 0.55) (layer F.Cu) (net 2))
 (segment (start 64.389 64.3128) (end 65.237528 64.3128) (width 0.55) (layer F.Cu) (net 2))
 (segment (start 68.8063 62.7634) (end 69.1134 63.0705) (width 0.55) (layer F.Cu) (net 4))
 (segment (start 64.389 62.7634) (end 64.389 62.7634) (width 0.55) (layer F.Cu) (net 4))
 (segment (start 72.2099 63.0705) (end 72.3646 62.9158) (width 0.55) (layer F.Cu) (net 4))
 (segment (start 69.1134 63.0705) (end 72.2099 63.0705) (width 0.55) (layer F.Cu) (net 4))
 (segment (start 87.44698 63.17969) (end 89.47249 63.17969) (width 0.55) (layer F.Cu) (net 4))
 (segment (start 87.18309 62.9158) (end 87.44698 63.17969) (width 0.55) (layer F.Cu) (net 4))
 (segment (start 89.47249 63.17969) (end 89.8182 63.5254) (width 0.55) (layer F.Cu) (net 4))
 (segment (start 72.3646 62.9158) (end 87.18309 62.9158) (width 0.55) (layer F.Cu) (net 4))
 (segment (start 84.2264 63.5254) (end 89.8182 63.5254) (width 0.55) (layer F.Cu) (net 4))
 (segment (start 82.2706 65.4812) (end 84.2264 63.5254) (width 0.55) (layer F.Cu) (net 4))
 (segment (start 64.389 62.7634) (end 68.8063 62.7634) (width 0.55) (layer F.Cu) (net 4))
 (segment (start 69.1365 61.214) (end 69.1642 61.1863) (width 0.55) (layer F.Cu) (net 3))
 (segment (start 64.389 61.214) (end 64.389 61.214) (width 0.55) (layer F.Cu) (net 3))
 (segment (start 72.3392 61.1863) (end 69.1642 61.1863) (width 0.55) (layer F.Cu) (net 3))
 (segment (start 88.7491 61.1863) (end 89.8182 62.2554) (width 0.55) (layer F.Cu) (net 3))
 (segment (start 82.3237 61.1863) (end 88.7491 61.1863) (width 0.55) (layer F.Cu) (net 3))
 (segment (start 72.3392 61.1863) (end 82.3237 61.1863) (width 0.55) (layer F.Cu) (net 3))
 (segment (start 82.1944 61.057) (end 82.3237 61.1863) (width 0.55) (layer F.Cu) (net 3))
 (segment (start 82.1944 59.2074) (end 82.1944 61.057) (width 0.55) (layer F.Cu) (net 3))
 (segment (start 64.389 61.214) (end 69.1365 61.214) (width 0.55) (layer F.Cu) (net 3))
 (segment (start 102.4382 63.5254) (end 102.9208 63.0428) (width 0.55) (layer F.Cu) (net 8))
 (segment (start 99.8182 63.5254) (end 102.4382 63.5254) (width 0.55) (layer F.Cu) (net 8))
 (segment (start 102.38479 70.59539) (end 102.613528 70.824128) (width 0.25) (layer F.Cu) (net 11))
 (segment (start 100.53819 70.59539) (end 102.38479 70.59539) (width 0.25) (layer F.Cu) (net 11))
 (segment (start 102.613528 70.824128) (end 103.1126 71.3232) (width 0.25) (layer F.Cu) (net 11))
 (segment (start 99.8182 69.8754) (end 100.53819 70.59539) (width 0.25) (layer F.Cu) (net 11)))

